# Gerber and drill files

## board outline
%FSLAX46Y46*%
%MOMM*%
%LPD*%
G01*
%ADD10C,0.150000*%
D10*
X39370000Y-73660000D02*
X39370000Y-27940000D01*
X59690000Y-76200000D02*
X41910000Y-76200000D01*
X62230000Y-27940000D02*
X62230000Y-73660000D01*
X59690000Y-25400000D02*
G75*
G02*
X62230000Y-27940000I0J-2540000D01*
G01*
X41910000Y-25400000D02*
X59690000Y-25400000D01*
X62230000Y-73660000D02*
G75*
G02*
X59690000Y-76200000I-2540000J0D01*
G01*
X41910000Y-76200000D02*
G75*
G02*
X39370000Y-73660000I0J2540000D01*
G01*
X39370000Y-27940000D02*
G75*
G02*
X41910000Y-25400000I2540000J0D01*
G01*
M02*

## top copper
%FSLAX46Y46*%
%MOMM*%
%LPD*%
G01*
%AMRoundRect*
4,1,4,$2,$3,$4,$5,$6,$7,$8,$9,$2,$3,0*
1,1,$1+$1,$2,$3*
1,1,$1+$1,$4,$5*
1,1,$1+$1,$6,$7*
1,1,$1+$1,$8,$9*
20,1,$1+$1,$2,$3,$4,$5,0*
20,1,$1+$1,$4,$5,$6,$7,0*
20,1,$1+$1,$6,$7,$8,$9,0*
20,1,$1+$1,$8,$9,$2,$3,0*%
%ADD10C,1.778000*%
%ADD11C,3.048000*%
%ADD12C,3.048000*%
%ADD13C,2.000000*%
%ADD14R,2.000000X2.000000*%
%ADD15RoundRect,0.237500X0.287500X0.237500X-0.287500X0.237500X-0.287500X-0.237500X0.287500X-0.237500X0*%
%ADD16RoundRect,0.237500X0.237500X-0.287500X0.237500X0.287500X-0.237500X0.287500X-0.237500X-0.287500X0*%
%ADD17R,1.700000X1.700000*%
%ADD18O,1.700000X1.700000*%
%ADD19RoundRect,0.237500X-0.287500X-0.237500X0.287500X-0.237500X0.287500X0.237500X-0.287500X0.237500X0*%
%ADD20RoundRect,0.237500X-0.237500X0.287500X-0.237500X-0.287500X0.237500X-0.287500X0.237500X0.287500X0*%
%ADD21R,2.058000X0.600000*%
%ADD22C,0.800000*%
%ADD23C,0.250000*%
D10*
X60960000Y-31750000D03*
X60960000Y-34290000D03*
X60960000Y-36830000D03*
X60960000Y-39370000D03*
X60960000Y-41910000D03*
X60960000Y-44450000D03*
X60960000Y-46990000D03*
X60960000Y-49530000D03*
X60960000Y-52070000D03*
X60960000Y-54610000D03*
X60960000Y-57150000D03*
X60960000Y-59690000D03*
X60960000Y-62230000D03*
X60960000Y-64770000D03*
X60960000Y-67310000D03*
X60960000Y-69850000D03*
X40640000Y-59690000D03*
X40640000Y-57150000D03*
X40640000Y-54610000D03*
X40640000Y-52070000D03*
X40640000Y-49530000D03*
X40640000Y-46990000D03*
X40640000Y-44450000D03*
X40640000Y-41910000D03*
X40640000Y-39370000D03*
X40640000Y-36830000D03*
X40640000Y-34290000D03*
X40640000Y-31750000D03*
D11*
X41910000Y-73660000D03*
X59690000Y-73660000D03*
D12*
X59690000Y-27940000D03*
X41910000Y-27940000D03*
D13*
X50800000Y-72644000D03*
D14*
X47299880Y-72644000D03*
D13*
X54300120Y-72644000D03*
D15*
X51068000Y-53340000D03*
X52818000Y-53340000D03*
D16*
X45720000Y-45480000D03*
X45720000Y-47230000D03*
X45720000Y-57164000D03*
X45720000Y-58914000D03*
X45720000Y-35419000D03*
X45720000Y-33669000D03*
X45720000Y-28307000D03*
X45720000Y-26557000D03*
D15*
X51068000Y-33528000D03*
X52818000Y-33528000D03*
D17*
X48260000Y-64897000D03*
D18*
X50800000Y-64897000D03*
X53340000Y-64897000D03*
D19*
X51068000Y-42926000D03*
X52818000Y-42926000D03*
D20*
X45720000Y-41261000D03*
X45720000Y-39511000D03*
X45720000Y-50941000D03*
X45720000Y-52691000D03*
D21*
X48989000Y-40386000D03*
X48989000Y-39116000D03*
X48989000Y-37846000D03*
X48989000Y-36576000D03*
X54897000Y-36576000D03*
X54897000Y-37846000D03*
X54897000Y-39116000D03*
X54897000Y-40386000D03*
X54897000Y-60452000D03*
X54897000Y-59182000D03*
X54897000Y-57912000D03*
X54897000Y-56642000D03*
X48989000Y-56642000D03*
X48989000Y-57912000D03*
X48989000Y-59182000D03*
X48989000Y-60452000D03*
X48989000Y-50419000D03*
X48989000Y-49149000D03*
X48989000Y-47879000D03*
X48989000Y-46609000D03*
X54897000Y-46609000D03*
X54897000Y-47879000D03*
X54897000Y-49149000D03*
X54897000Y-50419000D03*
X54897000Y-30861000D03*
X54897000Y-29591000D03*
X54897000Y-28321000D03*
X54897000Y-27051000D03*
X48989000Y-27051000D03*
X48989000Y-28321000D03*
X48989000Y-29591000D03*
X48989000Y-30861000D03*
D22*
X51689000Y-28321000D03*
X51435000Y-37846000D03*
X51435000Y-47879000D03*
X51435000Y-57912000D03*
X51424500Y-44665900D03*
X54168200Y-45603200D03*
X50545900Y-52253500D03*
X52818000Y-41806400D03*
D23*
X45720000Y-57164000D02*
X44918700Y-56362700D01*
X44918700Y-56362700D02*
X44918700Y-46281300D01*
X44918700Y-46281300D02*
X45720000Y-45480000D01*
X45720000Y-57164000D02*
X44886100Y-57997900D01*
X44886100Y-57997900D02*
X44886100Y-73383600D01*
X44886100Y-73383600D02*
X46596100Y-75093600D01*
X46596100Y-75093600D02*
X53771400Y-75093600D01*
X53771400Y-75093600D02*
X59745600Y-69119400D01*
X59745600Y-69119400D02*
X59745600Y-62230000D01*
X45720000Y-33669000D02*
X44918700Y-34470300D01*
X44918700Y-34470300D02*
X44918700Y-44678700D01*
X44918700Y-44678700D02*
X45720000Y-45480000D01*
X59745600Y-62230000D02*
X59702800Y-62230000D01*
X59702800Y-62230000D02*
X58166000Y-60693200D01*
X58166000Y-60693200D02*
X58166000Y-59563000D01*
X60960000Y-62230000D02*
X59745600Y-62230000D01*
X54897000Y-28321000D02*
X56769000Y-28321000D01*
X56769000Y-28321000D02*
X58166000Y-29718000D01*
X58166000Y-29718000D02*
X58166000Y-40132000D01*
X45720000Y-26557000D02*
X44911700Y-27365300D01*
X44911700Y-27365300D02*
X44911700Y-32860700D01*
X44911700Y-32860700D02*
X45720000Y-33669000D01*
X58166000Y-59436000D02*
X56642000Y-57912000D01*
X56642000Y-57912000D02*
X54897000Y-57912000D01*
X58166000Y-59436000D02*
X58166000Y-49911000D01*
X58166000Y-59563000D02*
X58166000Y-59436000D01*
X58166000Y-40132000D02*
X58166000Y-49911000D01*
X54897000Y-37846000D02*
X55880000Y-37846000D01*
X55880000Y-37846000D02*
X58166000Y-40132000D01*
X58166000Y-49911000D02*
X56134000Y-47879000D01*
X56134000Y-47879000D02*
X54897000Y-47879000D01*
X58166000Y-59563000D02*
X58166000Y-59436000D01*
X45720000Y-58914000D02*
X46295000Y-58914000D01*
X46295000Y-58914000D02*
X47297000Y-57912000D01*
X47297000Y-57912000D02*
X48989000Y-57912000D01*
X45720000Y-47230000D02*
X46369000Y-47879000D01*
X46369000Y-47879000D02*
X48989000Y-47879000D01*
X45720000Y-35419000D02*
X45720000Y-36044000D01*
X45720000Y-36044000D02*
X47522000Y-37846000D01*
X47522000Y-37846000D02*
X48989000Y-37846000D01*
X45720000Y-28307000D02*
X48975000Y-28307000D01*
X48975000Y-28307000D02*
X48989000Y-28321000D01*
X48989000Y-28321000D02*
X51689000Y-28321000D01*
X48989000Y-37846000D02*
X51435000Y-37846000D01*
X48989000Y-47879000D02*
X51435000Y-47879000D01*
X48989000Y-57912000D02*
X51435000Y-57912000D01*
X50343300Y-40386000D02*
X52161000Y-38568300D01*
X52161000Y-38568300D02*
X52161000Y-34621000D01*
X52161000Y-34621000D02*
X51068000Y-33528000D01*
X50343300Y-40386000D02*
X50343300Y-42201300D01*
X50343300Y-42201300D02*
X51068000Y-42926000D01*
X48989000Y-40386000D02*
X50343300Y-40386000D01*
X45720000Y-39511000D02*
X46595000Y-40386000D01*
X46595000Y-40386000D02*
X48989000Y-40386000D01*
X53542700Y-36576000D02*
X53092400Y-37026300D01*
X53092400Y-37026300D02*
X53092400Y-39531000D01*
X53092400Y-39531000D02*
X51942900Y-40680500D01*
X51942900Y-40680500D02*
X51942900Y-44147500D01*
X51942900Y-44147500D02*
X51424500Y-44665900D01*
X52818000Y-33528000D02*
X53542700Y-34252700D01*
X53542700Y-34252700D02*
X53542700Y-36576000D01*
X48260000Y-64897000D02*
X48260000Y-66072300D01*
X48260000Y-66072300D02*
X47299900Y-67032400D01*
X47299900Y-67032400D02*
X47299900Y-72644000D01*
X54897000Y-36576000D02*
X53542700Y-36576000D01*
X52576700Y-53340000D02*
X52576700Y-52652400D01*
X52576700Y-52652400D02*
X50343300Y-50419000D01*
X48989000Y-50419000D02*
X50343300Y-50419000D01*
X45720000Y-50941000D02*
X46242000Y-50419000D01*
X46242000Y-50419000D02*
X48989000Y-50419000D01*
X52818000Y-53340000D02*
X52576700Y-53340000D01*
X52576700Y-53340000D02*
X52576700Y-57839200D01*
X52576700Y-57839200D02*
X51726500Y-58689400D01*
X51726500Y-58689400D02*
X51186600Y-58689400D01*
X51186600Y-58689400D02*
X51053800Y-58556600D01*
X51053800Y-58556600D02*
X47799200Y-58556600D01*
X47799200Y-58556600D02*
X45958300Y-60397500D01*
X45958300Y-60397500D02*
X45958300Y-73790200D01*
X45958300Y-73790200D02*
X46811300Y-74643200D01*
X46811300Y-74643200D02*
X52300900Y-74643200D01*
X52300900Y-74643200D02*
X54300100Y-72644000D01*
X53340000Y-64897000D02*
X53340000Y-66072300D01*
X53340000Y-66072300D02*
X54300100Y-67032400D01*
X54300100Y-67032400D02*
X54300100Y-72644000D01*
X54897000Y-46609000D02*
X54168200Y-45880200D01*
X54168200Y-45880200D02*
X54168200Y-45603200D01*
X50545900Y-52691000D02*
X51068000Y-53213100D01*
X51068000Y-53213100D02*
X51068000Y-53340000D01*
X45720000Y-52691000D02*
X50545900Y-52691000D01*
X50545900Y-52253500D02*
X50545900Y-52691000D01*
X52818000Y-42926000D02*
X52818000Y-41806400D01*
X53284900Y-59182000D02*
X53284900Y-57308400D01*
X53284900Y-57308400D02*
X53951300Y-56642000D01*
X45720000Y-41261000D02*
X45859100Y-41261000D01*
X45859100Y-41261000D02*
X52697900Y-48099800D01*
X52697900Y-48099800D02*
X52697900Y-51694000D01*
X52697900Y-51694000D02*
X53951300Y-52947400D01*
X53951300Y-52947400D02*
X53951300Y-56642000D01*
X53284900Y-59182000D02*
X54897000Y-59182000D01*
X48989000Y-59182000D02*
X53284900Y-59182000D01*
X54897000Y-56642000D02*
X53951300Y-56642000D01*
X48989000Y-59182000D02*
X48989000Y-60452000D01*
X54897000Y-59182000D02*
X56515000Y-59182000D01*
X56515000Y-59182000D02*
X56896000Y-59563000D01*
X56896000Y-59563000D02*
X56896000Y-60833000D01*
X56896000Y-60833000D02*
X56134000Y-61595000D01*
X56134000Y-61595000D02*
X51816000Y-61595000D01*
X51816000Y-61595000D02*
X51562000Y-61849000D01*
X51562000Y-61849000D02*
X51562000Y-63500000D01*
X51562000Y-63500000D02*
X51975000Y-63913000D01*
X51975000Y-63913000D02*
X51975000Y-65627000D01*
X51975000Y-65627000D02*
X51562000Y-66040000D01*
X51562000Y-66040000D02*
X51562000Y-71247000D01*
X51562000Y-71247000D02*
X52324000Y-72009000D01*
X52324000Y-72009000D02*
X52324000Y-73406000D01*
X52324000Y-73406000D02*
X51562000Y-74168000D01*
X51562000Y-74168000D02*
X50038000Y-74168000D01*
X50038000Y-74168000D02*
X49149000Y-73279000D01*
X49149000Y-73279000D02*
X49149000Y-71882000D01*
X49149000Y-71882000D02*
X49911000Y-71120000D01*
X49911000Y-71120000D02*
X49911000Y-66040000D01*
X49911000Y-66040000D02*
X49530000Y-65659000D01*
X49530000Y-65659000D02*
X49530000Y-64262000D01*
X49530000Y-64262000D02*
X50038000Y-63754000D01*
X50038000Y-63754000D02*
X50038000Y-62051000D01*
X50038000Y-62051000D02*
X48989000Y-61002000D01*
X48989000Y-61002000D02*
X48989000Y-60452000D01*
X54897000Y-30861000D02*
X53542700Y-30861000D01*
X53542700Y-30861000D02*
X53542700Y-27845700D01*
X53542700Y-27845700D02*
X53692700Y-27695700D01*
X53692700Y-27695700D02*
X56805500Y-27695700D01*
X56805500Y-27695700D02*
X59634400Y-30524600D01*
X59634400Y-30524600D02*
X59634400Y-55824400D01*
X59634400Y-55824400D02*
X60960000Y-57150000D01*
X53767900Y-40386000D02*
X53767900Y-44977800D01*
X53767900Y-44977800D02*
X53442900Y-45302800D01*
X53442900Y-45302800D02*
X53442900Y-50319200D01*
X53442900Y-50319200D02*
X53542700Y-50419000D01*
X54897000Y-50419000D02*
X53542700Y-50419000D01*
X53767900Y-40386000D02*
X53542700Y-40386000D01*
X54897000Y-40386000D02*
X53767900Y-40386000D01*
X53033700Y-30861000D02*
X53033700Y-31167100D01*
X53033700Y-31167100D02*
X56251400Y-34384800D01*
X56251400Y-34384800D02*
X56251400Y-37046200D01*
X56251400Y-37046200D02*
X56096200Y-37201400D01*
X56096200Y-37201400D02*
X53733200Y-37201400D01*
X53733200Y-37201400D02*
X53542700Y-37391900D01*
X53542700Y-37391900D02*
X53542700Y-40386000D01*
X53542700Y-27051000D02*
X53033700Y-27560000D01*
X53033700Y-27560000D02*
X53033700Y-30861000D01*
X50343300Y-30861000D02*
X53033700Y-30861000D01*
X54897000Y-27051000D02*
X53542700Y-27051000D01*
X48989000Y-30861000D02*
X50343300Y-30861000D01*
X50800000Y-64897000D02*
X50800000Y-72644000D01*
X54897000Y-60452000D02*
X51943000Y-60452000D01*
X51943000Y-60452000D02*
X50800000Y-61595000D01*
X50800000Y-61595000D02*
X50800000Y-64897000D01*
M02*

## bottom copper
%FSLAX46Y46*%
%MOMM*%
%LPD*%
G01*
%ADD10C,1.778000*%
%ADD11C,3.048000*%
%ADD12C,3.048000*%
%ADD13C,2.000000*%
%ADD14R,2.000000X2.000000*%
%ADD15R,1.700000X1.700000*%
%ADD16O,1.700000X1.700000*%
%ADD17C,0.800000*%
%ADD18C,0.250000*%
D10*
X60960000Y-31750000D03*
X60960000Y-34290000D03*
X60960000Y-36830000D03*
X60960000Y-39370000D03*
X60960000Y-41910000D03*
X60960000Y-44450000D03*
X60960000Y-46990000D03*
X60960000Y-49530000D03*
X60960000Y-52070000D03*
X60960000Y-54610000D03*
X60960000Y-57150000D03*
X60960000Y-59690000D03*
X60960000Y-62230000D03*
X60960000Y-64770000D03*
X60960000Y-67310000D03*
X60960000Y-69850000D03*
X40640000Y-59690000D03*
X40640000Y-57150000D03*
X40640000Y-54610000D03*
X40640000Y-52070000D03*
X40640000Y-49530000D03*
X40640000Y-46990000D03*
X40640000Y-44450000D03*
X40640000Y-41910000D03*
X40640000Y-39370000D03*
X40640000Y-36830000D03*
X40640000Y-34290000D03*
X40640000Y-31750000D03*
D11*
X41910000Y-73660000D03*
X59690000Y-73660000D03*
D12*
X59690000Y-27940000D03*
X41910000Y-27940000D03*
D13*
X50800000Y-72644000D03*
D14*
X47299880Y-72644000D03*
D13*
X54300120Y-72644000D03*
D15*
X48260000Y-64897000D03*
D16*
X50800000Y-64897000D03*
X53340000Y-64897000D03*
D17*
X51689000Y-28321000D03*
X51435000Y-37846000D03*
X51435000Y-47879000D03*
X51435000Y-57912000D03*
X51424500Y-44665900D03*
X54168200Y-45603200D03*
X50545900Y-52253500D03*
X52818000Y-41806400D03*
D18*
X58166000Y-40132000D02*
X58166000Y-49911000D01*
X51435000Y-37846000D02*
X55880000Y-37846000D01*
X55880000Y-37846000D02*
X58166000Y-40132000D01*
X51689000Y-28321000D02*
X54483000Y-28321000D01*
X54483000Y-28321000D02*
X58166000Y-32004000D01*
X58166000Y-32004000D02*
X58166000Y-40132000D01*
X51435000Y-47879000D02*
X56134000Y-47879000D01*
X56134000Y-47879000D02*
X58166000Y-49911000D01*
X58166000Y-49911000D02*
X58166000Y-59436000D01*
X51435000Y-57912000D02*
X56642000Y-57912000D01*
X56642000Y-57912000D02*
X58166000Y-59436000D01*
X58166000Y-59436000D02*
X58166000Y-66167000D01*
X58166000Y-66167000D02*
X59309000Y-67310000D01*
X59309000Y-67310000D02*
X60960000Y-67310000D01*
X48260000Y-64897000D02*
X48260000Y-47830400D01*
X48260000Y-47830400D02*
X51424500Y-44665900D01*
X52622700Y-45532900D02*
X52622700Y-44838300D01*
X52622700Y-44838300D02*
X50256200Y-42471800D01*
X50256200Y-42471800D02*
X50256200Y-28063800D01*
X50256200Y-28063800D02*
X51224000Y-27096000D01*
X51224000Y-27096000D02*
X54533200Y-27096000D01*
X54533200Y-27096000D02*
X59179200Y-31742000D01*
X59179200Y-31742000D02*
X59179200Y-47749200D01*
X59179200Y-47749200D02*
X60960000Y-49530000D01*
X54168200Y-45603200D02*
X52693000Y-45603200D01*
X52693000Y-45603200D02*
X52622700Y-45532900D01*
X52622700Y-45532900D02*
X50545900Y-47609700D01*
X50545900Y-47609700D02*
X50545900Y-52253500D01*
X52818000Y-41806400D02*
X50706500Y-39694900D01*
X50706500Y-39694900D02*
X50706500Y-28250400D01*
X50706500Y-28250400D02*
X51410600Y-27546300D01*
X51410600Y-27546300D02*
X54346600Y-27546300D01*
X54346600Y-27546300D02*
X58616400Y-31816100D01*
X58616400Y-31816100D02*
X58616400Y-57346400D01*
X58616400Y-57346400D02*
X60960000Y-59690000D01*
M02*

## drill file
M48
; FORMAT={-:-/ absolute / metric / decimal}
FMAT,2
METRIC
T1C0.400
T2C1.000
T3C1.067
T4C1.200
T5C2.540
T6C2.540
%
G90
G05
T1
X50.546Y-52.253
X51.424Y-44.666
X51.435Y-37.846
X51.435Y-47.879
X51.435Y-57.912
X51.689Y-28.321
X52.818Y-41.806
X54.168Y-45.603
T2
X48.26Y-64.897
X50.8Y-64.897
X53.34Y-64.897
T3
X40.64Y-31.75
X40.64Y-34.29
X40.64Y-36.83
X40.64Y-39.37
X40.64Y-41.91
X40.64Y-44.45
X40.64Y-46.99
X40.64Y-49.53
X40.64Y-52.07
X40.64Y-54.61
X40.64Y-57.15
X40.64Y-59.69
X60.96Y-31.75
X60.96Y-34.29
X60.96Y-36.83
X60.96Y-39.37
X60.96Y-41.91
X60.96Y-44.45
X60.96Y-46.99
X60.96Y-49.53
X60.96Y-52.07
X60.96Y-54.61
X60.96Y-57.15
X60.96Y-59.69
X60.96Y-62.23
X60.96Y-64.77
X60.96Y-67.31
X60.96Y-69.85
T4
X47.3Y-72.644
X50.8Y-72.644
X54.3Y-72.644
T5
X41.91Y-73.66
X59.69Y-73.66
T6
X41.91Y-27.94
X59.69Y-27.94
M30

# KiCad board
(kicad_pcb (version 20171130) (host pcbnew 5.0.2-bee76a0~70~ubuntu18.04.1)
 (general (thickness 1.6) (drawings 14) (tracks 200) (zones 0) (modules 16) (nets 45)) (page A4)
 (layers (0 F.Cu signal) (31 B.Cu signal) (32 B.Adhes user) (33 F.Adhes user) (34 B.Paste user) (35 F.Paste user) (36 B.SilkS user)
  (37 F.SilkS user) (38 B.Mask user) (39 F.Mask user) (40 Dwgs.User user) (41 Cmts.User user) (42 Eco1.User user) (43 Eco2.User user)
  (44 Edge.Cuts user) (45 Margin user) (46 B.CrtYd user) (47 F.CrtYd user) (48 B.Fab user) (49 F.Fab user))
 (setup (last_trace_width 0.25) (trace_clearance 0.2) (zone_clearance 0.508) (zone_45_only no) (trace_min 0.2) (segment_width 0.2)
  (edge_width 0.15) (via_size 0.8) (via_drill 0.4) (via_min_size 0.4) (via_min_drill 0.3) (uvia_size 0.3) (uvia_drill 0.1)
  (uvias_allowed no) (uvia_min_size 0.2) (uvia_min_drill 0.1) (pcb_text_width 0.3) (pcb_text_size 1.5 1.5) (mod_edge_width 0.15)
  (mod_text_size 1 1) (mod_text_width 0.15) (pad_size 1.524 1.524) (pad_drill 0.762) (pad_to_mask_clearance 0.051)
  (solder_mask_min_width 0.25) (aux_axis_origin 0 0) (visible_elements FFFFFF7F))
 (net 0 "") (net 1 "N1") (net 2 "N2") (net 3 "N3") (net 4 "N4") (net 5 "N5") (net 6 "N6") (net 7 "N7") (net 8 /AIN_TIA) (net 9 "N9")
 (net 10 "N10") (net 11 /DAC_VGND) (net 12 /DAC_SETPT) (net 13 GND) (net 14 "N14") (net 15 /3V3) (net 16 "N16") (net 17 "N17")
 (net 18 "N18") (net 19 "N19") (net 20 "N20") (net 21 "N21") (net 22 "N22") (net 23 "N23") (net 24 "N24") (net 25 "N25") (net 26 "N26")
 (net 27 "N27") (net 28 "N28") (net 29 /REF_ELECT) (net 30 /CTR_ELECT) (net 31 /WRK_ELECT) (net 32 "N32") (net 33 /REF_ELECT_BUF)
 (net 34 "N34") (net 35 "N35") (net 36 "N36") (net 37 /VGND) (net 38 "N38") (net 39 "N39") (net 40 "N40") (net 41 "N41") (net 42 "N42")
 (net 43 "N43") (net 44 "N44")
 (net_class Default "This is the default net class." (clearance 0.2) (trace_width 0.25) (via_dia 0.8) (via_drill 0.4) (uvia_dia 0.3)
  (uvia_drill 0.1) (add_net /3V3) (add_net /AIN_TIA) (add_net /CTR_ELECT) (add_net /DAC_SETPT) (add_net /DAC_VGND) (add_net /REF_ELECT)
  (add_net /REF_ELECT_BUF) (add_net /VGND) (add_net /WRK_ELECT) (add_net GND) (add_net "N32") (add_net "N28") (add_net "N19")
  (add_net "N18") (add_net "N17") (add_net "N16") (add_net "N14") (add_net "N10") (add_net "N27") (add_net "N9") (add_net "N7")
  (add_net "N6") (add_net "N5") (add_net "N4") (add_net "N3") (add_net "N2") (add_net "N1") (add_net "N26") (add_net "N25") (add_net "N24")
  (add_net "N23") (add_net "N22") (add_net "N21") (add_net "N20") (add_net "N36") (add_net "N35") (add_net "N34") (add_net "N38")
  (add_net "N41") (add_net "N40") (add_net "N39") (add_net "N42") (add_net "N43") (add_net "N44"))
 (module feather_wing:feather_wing (layer F.Cu) (at 50.8 50.8)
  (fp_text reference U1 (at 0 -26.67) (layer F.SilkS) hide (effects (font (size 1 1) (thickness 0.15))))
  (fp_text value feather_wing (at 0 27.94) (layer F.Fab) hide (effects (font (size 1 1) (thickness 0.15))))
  (pad 28 thru_hole circle (at 10.16 -19.05) (size 1.778 1.778) (drill 1.0668) (layers *.Cu *.Mask) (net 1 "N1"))
  (pad 27 thru_hole circle (at 10.16 -16.51) (size 1.778 1.778) (drill 1.0668) (layers *.Cu *.Mask) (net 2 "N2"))
  (pad 26 thru_hole circle (at 10.16 -13.97) (size 1.778 1.778) (drill 1.0668) (layers *.Cu *.Mask) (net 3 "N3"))
  (pad 25 thru_hole circle (at 10.16 -11.43) (size 1.778 1.778) (drill 1.0668) (layers *.Cu *.Mask) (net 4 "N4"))
  (pad 24 thru_hole circle (at 10.16 -8.89) (size 1.778 1.778) (drill 1.0668) (layers *.Cu *.Mask) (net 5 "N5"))
  (pad 23 thru_hole circle (at 10.16 -6.35) (size 1.778 1.778) (drill 1.0668) (layers *.Cu *.Mask) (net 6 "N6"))
  (pad 22 thru_hole circle (at 10.16 -3.81) (size 1.778 1.778) (drill 1.0668) (layers *.Cu *.Mask) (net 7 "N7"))
  (pad 21 thru_hole circle (at 10.16 -1.27) (size 1.778 1.778) (drill 1.0668) (layers *.Cu *.Mask) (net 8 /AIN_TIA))
  (pad 20 thru_hole circle (at 10.16 1.27) (size 1.778 1.778) (drill 1.0668) (layers *.Cu *.Mask) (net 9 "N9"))
  (pad 19 thru_hole circle (at 10.16 3.81) (size 1.778 1.778) (drill 1.0668) (layers *.Cu *.Mask) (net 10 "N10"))
  (pad 18 thru_hole circle (at 10.16 6.35) (size 1.778 1.778) (drill 1.0668) (layers *.Cu *.Mask) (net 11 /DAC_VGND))
  (pad 17 thru_hole circle (at 10.16 8.89) (size 1.778 1.778) (drill 1.0668) (layers *.Cu *.Mask) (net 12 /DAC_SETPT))
  (pad 16 thru_hole circle (at 10.16 11.43) (size 1.778 1.778) (drill 1.0668) (layers *.Cu *.Mask) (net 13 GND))
  (pad 15 thru_hole circle (at 10.16 13.97) (size 1.778 1.778) (drill 1.0668) (layers *.Cu *.Mask) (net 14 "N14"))
  (pad 14 thru_hole circle (at 10.16 16.51) (size 1.778 1.778) (drill 1.0668) (layers *.Cu *.Mask) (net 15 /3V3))
  (pad 13 thru_hole circle (at 10.16 19.05) (size 1.778 1.778) (drill 1.0668) (layers *.Cu *.Mask) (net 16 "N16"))
  (pad 12 thru_hole circle (at -10.16 8.89) (size 1.778 1.778) (drill 1.0668) (layers *.Cu *.Mask) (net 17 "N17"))
  (pad 11 thru_hole circle (at -10.16 6.35) (size 1.778 1.778) (drill 1.0668) (layers *.Cu *.Mask) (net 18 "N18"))
  (pad 10 thru_hole circle (at -10.16 3.81) (size 1.778 1.778) (drill 1.0668) (layers *.Cu *.Mask) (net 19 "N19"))
  (pad 9 thru_hole circle (at -10.16 1.27) (size 1.778 1.778) (drill 1.0668) (layers *.Cu *.Mask) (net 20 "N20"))
  (pad 8 thru_hole circle (at -10.16 -1.27) (size 1.778 1.778) (drill 1.0668) (layers *.Cu *.Mask) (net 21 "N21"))
  (pad 7 thru_hole circle (at -10.16 -3.81) (size 1.778 1.778) (drill 1.0668) (layers *.Cu *.Mask) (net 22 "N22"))
  (pad 6 thru_hole circle (at -10.16 -6.35) (size 1.778 1.778) (drill 1.0668) (layers *.Cu *.Mask) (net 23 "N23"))
  (pad 5 thru_hole circle (at -10.16 -8.89) (size 1.778 1.778) (drill 1.0668) (layers *.Cu *.Mask) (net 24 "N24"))
  (pad 4 thru_hole circle (at -10.16 -11.43) (size 1.778 1.778) (drill 1.0668) (layers *.Cu *.Mask) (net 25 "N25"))
  (pad 3 thru_hole circle (at -10.16 -13.97) (size 1.778 1.778) (drill 1.0668) (layers *.Cu *.Mask) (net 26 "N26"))
  (pad 2 thru_hole circle (at -10.16 -16.51) (size 1.778 1.778) (drill 1.0668) (layers *.Cu *.Mask) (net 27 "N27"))
  (pad 1 thru_hole circle (at -10.16 -19.05) (size 1.778 1.778) (drill 1.0668) (layers *.Cu *.Mask) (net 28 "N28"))
  (pad "" thru_hole circle (at -8.89 22.86) (size 3.048 3.048) (drill 2.54) (layers *.Cu *.Mask))
  (pad "" thru_hole circle (at 8.89 22.86) (size 3.048 3.048) (drill 2.54) (layers *.Cu *.Mask))
  (pad "" np_thru_hole circle (at 8.89 -22.86) (size 3.048 3.048) (drill 2.54) (layers *.Cu *.Mask))
  (pad "" np_thru_hole circle (at -8.89 -22.86) (size 3.048 3.048) (drill 2.54) (layers *.Cu *.Mask)))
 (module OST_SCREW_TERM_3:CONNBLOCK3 (layer F.Cu) (at 50.8 72.644)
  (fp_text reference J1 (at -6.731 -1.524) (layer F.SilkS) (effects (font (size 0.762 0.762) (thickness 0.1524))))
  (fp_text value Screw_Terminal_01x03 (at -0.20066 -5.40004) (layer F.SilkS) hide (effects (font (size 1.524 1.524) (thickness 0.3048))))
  (pad 2 thru_hole circle (at 0 0) (size 2 2) (drill 1.2) (layers *.Cu *.Mask) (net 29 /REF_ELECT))
  (pad 1 thru_hole rect (at -3.50012 0) (size 2 2) (drill 1.2) (layers *.Cu *.Mask) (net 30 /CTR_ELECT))
  (pad 3 thru_hole circle (at 3.50012 0) (size 2 2) (drill 1.2) (layers *.Cu *.Mask) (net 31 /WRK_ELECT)))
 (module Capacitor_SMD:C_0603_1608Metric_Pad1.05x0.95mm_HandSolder (layer F.Cu) (at 51.943 53.34 180)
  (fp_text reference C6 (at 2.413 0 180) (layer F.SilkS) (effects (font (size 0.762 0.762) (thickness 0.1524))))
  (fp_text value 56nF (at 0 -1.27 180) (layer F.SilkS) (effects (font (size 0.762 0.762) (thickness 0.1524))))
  (pad 2 smd roundrect (at 0.875 0 180) (size 1.05 0.95) (layers F.Cu F.Paste F.Mask) (roundrect_rratio 0.25) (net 8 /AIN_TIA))
  (pad 1 smd roundrect (at -0.875 0 180) (size 1.05 0.95) (layers F.Cu F.Paste F.Mask) (roundrect_rratio 0.25) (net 31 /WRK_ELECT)))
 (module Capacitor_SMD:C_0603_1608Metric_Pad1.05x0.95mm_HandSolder (layer F.Cu) (at 45.72 46.355 90)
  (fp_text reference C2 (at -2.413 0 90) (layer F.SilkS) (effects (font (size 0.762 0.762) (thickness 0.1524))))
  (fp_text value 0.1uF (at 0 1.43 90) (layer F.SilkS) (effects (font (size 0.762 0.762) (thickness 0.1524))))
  (pad 2 smd roundrect (at 0.875 0 90) (size 1.05 0.95) (layers F.Cu F.Paste F.Mask) (roundrect_rratio 0.25) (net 13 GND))
  (pad 1 smd roundrect (at -0.875 0 90) (size 1.05 0.95) (layers F.Cu F.Paste F.Mask) (roundrect_rratio 0.25) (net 15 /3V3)))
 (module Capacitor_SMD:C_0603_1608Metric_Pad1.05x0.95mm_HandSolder (layer F.Cu) (at 45.72 58.039 90)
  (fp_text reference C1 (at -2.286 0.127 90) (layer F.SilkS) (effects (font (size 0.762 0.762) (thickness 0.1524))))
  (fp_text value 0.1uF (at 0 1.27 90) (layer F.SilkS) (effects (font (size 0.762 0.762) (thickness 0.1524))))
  (pad 2 smd roundrect (at 0.875 0 90) (size 1.05 0.95) (layers F.Cu F.Paste F.Mask) (roundrect_rratio 0.25) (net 13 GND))
  (pad 1 smd roundrect (at -0.875 0 90) (size 1.05 0.95) (layers F.Cu F.Paste F.Mask) (roundrect_rratio 0.25) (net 15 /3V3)))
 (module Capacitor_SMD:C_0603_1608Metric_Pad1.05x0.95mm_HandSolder (layer F.Cu) (at 45.72 34.544 90)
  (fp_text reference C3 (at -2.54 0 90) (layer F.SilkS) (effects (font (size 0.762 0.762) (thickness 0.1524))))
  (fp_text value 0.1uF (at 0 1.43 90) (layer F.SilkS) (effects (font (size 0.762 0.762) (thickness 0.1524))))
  (pad 1 smd roundrect (at -0.875 0 90) (size 1.05 0.95) (layers F.Cu F.Paste F.Mask) (roundrect_rratio 0.25) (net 15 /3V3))
  (pad 2 smd roundrect (at 0.875 0 90) (size 1.05 0.95) (layers F.Cu F.Paste F.Mask) (roundrect_rratio 0.25) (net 13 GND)))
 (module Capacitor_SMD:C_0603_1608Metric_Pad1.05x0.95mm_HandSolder (layer F.Cu) (at 45.72 27.432 90)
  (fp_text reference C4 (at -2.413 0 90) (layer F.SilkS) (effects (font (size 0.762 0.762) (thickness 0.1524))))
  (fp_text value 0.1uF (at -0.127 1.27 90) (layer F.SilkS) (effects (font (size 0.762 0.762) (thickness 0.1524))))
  (pad 1 smd roundrect (at -0.875 0 90) (size 1.05 0.95) (layers F.Cu F.Paste F.Mask) (roundrect_rratio 0.25) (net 15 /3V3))
  (pad 2 smd roundrect (at 0.875 0 90) (size 1.05 0.95) (layers F.Cu F.Paste F.Mask) (roundrect_rratio 0.25) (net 13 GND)))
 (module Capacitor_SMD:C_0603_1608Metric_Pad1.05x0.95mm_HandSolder (layer F.Cu) (at 51.943 33.528 180)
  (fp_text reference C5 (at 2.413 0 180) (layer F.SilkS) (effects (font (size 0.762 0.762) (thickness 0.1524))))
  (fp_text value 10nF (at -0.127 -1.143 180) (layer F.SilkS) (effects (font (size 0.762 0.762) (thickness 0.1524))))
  (pad 2 smd roundrect (at 0.875 0 180) (size 1.05 0.95) (layers F.Cu F.Paste F.Mask) (roundrect_rratio 0.25) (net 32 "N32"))
  (pad 1 smd roundrect (at -0.875 0 180) (size 1.05 0.95) (layers F.Cu F.Paste F.Mask) (roundrect_rratio 0.25) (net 30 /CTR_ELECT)))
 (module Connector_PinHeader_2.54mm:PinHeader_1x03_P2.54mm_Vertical (layer F.Cu) (at 48.26 64.897 90)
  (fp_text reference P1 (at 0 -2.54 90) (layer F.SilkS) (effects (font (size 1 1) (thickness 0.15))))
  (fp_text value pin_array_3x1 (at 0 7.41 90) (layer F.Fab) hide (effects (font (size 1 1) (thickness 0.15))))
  (pad 1 thru_hole rect (at 0 0 90) (size 1.7 1.7) (drill 1) (layers *.Cu *.Mask) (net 30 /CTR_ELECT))
  (pad 2 thru_hole oval (at 0 2.54 90) (size 1.7 1.7) (drill 1) (layers *.Cu *.Mask) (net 29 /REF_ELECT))
  (pad 3 thru_hole oval (at 0 5.08 90) (size 1.7 1.7) (drill 1) (layers *.Cu *.Mask) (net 31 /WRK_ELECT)))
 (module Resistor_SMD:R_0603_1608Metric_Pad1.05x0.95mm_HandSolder (layer F.Cu) (at 51.943 42.926)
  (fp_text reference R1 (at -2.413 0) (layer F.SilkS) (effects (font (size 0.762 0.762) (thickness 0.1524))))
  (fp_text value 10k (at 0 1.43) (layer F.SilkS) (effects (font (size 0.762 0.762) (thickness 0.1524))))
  (pad 1 smd roundrect (at -0.875 0) (size 1.05 0.95) (layers F.Cu F.Paste F.Mask) (roundrect_rratio 0.25) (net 32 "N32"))
  (pad 2 smd roundrect (at 0.875 0) (size 1.05 0.95) (layers F.Cu F.Paste F.Mask) (roundrect_rratio 0.25) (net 12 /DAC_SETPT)))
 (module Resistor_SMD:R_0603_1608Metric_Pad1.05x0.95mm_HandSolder (layer F.Cu) (at 45.72 40.386 270)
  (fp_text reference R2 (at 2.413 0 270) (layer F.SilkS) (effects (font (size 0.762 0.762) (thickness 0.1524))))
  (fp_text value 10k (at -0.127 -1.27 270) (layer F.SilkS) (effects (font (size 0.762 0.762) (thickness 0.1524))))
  (pad 2 smd roundrect (at 0.875 0 270) (size 1.05 0.95) (layers F.Cu F.Paste F.Mask) (roundrect_rratio 0.25) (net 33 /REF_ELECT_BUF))
  (pad 1 smd roundrect (at -0.875 0 270) (size 1.05 0.95) (layers F.Cu F.Paste F.Mask) (roundrect_rratio 0.25) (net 32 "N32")))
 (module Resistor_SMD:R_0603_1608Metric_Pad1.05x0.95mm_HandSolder (layer F.Cu) (at 45.72 51.816 270)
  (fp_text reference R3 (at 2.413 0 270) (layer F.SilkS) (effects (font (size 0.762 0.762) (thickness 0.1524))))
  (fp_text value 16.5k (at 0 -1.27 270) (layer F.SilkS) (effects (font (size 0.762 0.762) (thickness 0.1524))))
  (pad 1 smd roundrect (at -0.875 0 270) (size 1.05 0.95) (layers F.Cu F.Paste F.Mask) (roundrect_rratio 0.25) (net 31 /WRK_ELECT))
  (pad 2 smd roundrect (at 0.875 0 270) (size 1.05 0.95) (layers F.Cu F.Paste F.Mask) (roundrect_rratio 0.25) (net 8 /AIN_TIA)))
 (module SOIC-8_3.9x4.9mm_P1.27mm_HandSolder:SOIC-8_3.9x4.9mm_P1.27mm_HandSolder (layer F.Cu) (at 51.943 38.481 180)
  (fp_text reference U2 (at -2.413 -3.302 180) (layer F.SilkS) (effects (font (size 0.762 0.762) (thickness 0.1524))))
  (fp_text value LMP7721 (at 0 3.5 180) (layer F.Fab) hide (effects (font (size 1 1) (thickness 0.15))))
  (pad 8 smd rect (at 2.954 -1.905 180) (size 2.058 0.6) (layers F.Cu F.Paste F.Mask) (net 32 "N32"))
  (pad 7 smd rect (at 2.954 -0.635 180) (size 2.058 0.6) (layers F.Cu F.Paste F.Mask) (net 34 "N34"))
  (pad 6 smd rect (at 2.954 0.635 180) (size 2.058 0.6) (layers F.Cu F.Paste F.Mask) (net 15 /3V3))
  (pad 5 smd rect (at 2.954 1.905 180) (size 2.058 0.6) (layers F.Cu F.Paste F.Mask) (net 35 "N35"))
  (pad 4 smd rect (at -2.954 1.905 180) (size 2.058 0.6) (layers F.Cu F.Paste F.Mask) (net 30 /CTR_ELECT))
  (pad 3 smd rect (at -2.954 0.635 180) (size 2.058 0.6) (layers F.Cu F.Paste F.Mask) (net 13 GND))
  (pad 2 smd rect (at -2.954 -0.635 180) (size 2.058 0.6) (layers F.Cu F.Paste F.Mask) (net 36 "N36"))
  (pad 1 smd rect (at -2.954 -1.905 180) (size 2.058 0.6) (layers F.Cu F.Paste F.Mask) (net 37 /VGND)))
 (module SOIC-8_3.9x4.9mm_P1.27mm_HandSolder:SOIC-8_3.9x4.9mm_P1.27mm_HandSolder (layer F.Cu) (at 51.943 58.547 180)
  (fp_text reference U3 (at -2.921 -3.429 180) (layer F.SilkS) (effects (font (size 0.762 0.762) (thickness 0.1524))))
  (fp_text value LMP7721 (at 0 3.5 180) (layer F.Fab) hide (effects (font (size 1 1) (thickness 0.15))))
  (pad 1 smd rect (at -2.954 -1.905 180) (size 2.058 0.6) (layers F.Cu F.Paste F.Mask) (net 29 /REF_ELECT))
  (pad 2 smd rect (at -2.954 -0.635 180) (size 2.058 0.6) (layers F.Cu F.Paste F.Mask) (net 33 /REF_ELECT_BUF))
  (pad 3 smd rect (at -2.954 0.635 180) (size 2.058 0.6) (layers F.Cu F.Paste F.Mask) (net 13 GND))
  (pad 4 smd rect (at -2.954 1.905 180) (size 2.058 0.6) (layers F.Cu F.Paste F.Mask) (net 33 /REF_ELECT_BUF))
  (pad 5 smd rect (at 2.954 1.905 180) (size 2.058 0.6) (layers F.Cu F.Paste F.Mask) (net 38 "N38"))
  (pad 6 smd rect (at 2.954 0.635 180) (size 2.058 0.6) (layers F.Cu F.Paste F.Mask) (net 15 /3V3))
  (pad 7 smd rect (at 2.954 -0.635 180) (size 2.058 0.6) (layers F.Cu F.Paste F.Mask) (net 33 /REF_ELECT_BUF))
  (pad 8 smd rect (at 2.954 -1.905 180) (size 2.058 0.6) (layers F.Cu F.Paste F.Mask) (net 33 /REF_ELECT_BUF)))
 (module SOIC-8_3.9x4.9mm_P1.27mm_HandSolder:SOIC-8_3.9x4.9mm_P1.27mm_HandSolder (layer F.Cu) (at 51.943 48.514 180)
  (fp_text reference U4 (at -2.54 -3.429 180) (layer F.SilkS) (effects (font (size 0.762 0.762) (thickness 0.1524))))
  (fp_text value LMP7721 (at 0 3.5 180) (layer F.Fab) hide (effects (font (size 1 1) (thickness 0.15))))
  (pad 8 smd rect (at 2.954 -1.905 180) (size 2.058 0.6) (layers F.Cu F.Paste F.Mask) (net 31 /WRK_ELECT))
  (pad 7 smd rect (at 2.954 -0.635 180) (size 2.058 0.6) (layers F.Cu F.Paste F.Mask) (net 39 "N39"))
  (pad 6 smd rect (at 2.954 0.635 180) (size 2.058 0.6) (layers F.Cu F.Paste F.Mask) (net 15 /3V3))
  (pad 5 smd rect (at 2.954 1.905 180) (size 2.058 0.6) (layers F.Cu F.Paste F.Mask) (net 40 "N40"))
  (pad 4 smd rect (at -2.954 1.905 180) (size 2.058 0.6) (layers F.Cu F.Paste F.Mask) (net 8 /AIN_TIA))
  (pad 3 smd rect (at -2.954 0.635 180) (size 2.058 0.6) (layers F.Cu F.Paste F.Mask) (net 13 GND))
  (pad 2 smd rect (at -2.954 -0.635 180) (size 2.058 0.6) (layers F.Cu F.Paste F.Mask) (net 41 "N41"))
  (pad 1 smd rect (at -2.954 -1.905 180) (size 2.058 0.6) (layers F.Cu F.Paste F.Mask) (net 37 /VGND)))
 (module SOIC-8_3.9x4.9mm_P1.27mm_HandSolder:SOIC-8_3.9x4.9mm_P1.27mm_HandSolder (layer F.Cu) (at 51.943 28.956 180)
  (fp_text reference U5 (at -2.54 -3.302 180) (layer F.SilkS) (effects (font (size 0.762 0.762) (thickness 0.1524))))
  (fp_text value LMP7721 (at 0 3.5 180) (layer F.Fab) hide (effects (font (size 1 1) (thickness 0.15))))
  (pad 1 smd rect (at -2.954 -1.905 180) (size 2.058 0.6) (layers F.Cu F.Paste F.Mask) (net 11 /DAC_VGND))
  (pad 2 smd rect (at -2.954 -0.635 180) (size 2.058 0.6) (layers F.Cu F.Paste F.Mask) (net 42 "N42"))
  (pad 3 smd rect (at -2.954 0.635 180) (size 2.058 0.6) (layers F.Cu F.Paste F.Mask) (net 13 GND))
  (pad 4 smd rect (at -2.954 1.905 180) (size 2.058 0.6) (layers F.Cu F.Paste F.Mask) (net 37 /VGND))
  (pad 5 smd rect (at 2.954 1.905 180) (size 2.058 0.6) (layers F.Cu F.Paste F.Mask) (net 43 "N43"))
  (pad 6 smd rect (at 2.954 0.635 180) (size 2.058 0.6) (layers F.Cu F.Paste F.Mask) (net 15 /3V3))
  (pad 7 smd rect (at 2.954 -0.635 180) (size 2.058 0.6) (layers F.Cu F.Paste F.Mask) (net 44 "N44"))
  (pad 8 smd rect (at 2.954 -1.905 180) (size 2.058 0.6) (layers F.Cu F.Paste F.Mask) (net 37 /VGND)))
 (gr_line (start 39.37 73.66) (end 39.37 27.94) (layer Edge.Cuts) (width 0.15))
 (gr_line (start 59.69 76.2) (end 41.91 76.2) (layer Edge.Cuts) (width 0.15))
 (gr_line (start 62.23 27.94) (end 62.23 73.66) (layer Edge.Cuts) (width 0.15))
 (gr_arc (start 59.69 27.94) (end 62.23 27.94) (angle -90) (layer Edge.Cuts) (width 0.15))
 (gr_line (start 41.91 25.4) (end 59.69 25.4) (layer Edge.Cuts) (width 0.15))
 (gr_arc (start 59.69 73.66) (end 59.69 76.2) (angle -90) (layer Edge.Cuts) (width 0.15))
 (gr_arc (start 41.91 73.66) (end 39.37 73.66) (angle -90) (layer Edge.Cuts) (width 0.15))
 (gr_arc (start 41.91 27.94) (end 41.91 25.4) (angle -90) (layer Edge.Cuts) (width 0.15))
 (segment (start 45.72 57.164) (end 44.9187 56.3627) (width 0.25) (layer F.Cu) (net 13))
 (segment (start 44.9187 56.3627) (end 44.9187 46.2813) (width 0.25) (layer F.Cu) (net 13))
 (segment (start 44.9187 46.2813) (end 45.72 45.48) (width 0.25) (layer F.Cu) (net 13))
 (segment (start 45.72 57.164) (end 44.8861 57.9979) (width 0.25) (layer F.Cu) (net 13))
 (segment (start 44.8861 57.9979) (end 44.8861 73.3836) (width 0.25) (layer F.Cu) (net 13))
 (segment (start 44.8861 73.3836) (end 46.5961 75.0936) (width 0.25) (layer F.Cu) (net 13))
 (segment (start 46.5961 75.0936) (end 53.7714 75.0936) (width 0.25) (layer F.Cu) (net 13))
 (segment (start 53.7714 75.0936) (end 59.7456 69.1194) (width 0.25) (layer F.Cu) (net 13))
 (segment (start 59.7456 69.1194) (end 59.7456 62.23) (width 0.25) (layer F.Cu) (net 13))
 (segment (start 45.72 33.669) (end 44.9187 34.4703) (width 0.25) (layer F.Cu) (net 13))
 (segment (start 44.9187 34.4703) (end 44.9187 44.6787) (width 0.25) (layer F.Cu) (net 13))
 (segment (start 44.9187 44.6787) (end 45.72 45.48) (width 0.25) (layer F.Cu) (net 13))
 (segment (start 59.7456 62.23) (end 59.7028 62.23) (width 0.25) (layer F.Cu) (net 13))
 (segment (start 59.7028 62.23) (end 58.166 60.6932) (width 0.25) (layer F.Cu) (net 13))
 (segment (start 58.166 60.6932) (end 58.166 59.563) (width 0.25) (layer F.Cu) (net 13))
 (segment (start 60.96 62.23) (end 59.7456 62.23) (width 0.25) (layer F.Cu) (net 13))
 (segment (start 54.897 28.321) (end 56.769 28.321) (width 0.25) (layer F.Cu) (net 13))
 (segment (start 56.769 28.321) (end 58.166 29.718) (width 0.25) (layer F.Cu) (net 13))
 (segment (start 58.166 29.718) (end 58.166 40.132) (width 0.25) (layer F.Cu) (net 13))
 (segment (start 45.72 26.557) (end 44.9117 27.3653) (width 0.25) (layer F.Cu) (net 13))
 (segment (start 44.9117 27.3653) (end 44.9117 32.8607) (width 0.25) (layer F.Cu) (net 13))
 (segment (start 44.9117 32.8607) (end 45.72 33.669) (width 0.25) (layer F.Cu) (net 13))
 (segment (start 58.166 59.436) (end 56.642 57.912) (width 0.25) (layer F.Cu) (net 13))
 (segment (start 56.642 57.912) (end 54.897 57.912) (width 0.25) (layer F.Cu) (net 13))
 (segment (start 58.166 59.436) (end 58.166 49.911) (width 0.25) (layer F.Cu) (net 13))
 (segment (start 58.166 59.563) (end 58.166 59.436) (width 0.25) (layer F.Cu) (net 13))
 (segment (start 58.166 40.132) (end 58.166 49.911) (width 0.25) (layer F.Cu) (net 13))
 (segment (start 54.897 37.846) (end 55.88 37.846) (width 0.25) (layer F.Cu) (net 13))
 (segment (start 55.88 37.846) (end 58.166 40.132) (width 0.25) (layer F.Cu) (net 13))
 (segment (start 58.166 49.911) (end 56.134 47.879) (width 0.25) (layer F.Cu) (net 13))
 (segment (start 56.134 47.879) (end 54.897 47.879) (width 0.25) (layer F.Cu) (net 13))
 (segment (start 58.166 59.563) (end 58.166 59.436) (width 0.25) (layer F.Cu) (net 13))
 (segment (start 58.166 40.132) (end 58.166 49.911) (width 0.25) (layer B.Cu) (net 15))
 (segment (start 51.435 37.846) (end 55.88 37.846) (width 0.25) (layer B.Cu) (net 15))
 (segment (start 55.88 37.846) (end 58.166 40.132) (width 0.25) (layer B.Cu) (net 15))
 (segment (start 45.72 58.914) (end 46.295 58.914) (width 0.25) (layer F.Cu) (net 15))
 (segment (start 46.295 58.914) (end 47.297 57.912) (width 0.25) (layer F.Cu) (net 15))
 (segment (start 47.297 57.912) (end 48.989 57.912) (width 0.25) (layer F.Cu) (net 15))
 (segment (start 45.72 47.23) (end 46.369 47.879) (width 0.25) (layer F.Cu) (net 15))
 (segment (start 46.369 47.879) (end 48.989 47.879) (width 0.25) (layer F.Cu) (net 15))
 (segment (start 45.72 35.419) (end 45.72 36.044) (width 0.25) (layer F.Cu) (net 15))
 (segment (start 45.72 36.044) (end 47.522 37.846) (width 0.25) (layer F.Cu) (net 15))
 (segment (start 47.522 37.846) (end 48.989 37.846) (width 0.25) (layer F.Cu) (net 15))
 (segment (start 45.72 28.307) (end 48.975 28.307) (width 0.25) (layer F.Cu) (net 15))
 (segment (start 48.975 28.307) (end 48.989 28.321) (width 0.25) (layer F.Cu) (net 15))
 (segment (start 51.689 28.321) (end 54.483 28.321) (width 0.25) (layer B.Cu) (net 15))
 (segment (start 54.483 28.321) (end 58.166 32.004) (width 0.25) (layer B.Cu) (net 15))
 (segment (start 58.166 32.004) (end 58.166 40.132) (width 0.25) (layer B.Cu) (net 15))
 (segment (start 48.989 28.321) (end 51.689 28.321) (width 0.25) (layer F.Cu) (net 15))
 (segment (start 48.989 37.846) (end 51.435 37.846) (width 0.25) (layer F.Cu) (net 15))
 (segment (start 51.435 47.879) (end 56.134 47.879) (width 0.25) (layer B.Cu) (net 15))
 (segment (start 56.134 47.879) (end 58.166 49.911) (width 0.25) (layer B.Cu) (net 15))
 (segment (start 58.166 49.911) (end 58.166 59.436) (width 0.25) (layer B.Cu) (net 15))
 (segment (start 48.989 47.879) (end 51.435 47.879) (width 0.25) (layer F.Cu) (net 15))
 (segment (start 51.435 57.912) (end 56.642 57.912) (width 0.25) (layer B.Cu) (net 15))
 (segment (start 56.642 57.912) (end 58.166 59.436) (width 0.25) (layer B.Cu) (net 15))
 (segment (start 58.166 59.436) (end 58.166 66.167) (width 0.25) (layer B.Cu) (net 15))
 (segment (start 58.166 66.167) (end 59.309 67.31) (width 0.25) (layer B.Cu) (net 15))
 (segment (start 59.309 67.31) (end 60.96 67.31) (width 0.25) (layer B.Cu) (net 15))
 (segment (start 48.989 57.912) (end 51.435 57.912) (width 0.25) (layer F.Cu) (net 15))
 (via (at 51.689 28.321) (size 0.8) (layers F.Cu B.Cu) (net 15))
 (via (at 51.435 37.846) (size 0.8) (layers F.Cu B.Cu) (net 15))
 (via (at 51.435 47.879) (size 0.8) (layers F.Cu B.Cu) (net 15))
 (via (at 51.435 57.912) (size 0.8) (layers F.Cu B.Cu) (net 15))
 (segment (start 50.3433 40.386) (end 52.161 38.5683) (width 0.25) (layer F.Cu) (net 32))
 (segment (start 52.161 38.5683) (end 52.161 34.621) (width 0.25) (layer F.Cu) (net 32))
 (segment (start 52.161 34.621) (end 51.068 33.528) (width 0.25) (layer F.Cu) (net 32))
 (segment (start 50.3433 40.386) (end 50.3433 42.2013) (width 0.25) (layer F.Cu) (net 32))
 (segment (start 50.3433 42.2013) (end 51.068 42.926) (width 0.25) (layer F.Cu) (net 32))
 (segment (start 48.989 40.386) (end 50.3433 40.386) (width 0.25) (layer F.Cu) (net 32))
 (segment (start 45.72 39.511) (end 46.595 40.386) (width 0.25) (layer F.Cu) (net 32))
 (segment (start 46.595 40.386) (end 48.989 40.386) (width 0.25) (layer F.Cu) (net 32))
 (segment (start 53.5427 36.576) (end 53.0924 37.0263) (width 0.25) (layer F.Cu) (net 30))
 (segment (start 53.0924 37.0263) (end 53.0924 39.531) (width 0.25) (layer F.Cu) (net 30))
 (segment (start 53.0924 39.531) (end 51.9429 40.6805) (width 0.25) (layer F.Cu) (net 30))
 (segment (start 51.9429 40.6805) (end 51.9429 44.1475) (width 0.25) (layer F.Cu) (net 30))
 (segment (start 51.9429 44.1475) (end 51.4245 44.6659) (width 0.25) (layer F.Cu) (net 30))
 (segment (start 48.26 64.897) (end 48.26 47.8304) (width 0.25) (layer B.Cu) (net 30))
 (segment (start 48.26 47.8304) (end 51.4245 44.6659) (width 0.25) (layer B.Cu) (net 30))
 (segment (start 52.818 33.528) (end 53.5427 34.2527) (width 0.25) (layer F.Cu) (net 30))
 (segment (start 53.5427 34.2527) (end 53.5427 36.576) (width 0.25) (layer F.Cu) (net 30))
 (segment (start 48.26 64.897) (end 48.26 66.0723) (width 0.25) (layer F.Cu) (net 30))
 (segment (start 48.26 66.0723) (end 47.2999 67.0324) (width 0.25) (layer F.Cu) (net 30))
 (segment (start 47.2999 67.0324) (end 47.2999 72.644) (width 0.25) (layer F.Cu) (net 30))
 (segment (start 54.897 36.576) (end 53.5427 36.576) (width 0.25) (layer F.Cu) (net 30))
 (via (at 51.4245 44.6659) (size 0.8) (layers F.Cu B.Cu) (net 30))
 (segment (start 52.5767 53.34) (end 52.5767 52.6524) (width 0.25) (layer F.Cu) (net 31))
 (segment (start 52.5767 52.6524) (end 50.3433 50.419) (width 0.25) (layer F.Cu) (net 31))
 (segment (start 48.989 50.419) (end 50.3433 50.419) (width 0.25) (layer F.Cu) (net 31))
 (segment (start 45.72 50.941) (end 46.242 50.419) (width 0.25) (layer F.Cu) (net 31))
 (segment (start 46.242 50.419) (end 48.989 50.419) (width 0.25) (layer F.Cu) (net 31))
 (segment (start 52.818 53.34) (end 52.5767 53.34) (width 0.25) (layer F.Cu) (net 31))
 (segment (start 52.5767 53.34) (end 52.5767 57.8392) (width 0.25) (layer F.Cu) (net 31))
 (segment (start 52.5767 57.8392) (end 51.7265 58.6894) (width 0.25) (layer F.Cu) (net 31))
 (segment (start 51.7265 58.6894) (end 51.1866 58.6894) (width 0.25) (layer F.Cu) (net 31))
 (segment (start 51.1866 58.6894) (end 51.0538 58.5566) (width 0.25) (layer F.Cu) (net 31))
 (segment (start 51.0538 58.5566) (end 47.7992 58.5566) (width 0.25) (layer F.Cu) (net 31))
 (segment (start 47.7992 58.5566) (end 45.9583 60.3975) (width 0.25) (layer F.Cu) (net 31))
 (segment (start 45.9583 60.3975) (end 45.9583 73.7902) (width 0.25) (layer F.Cu) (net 31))
 (segment (start 45.9583 73.7902) (end 46.8113 74.6432) (width 0.25) (layer F.Cu) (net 31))
 (segment (start 46.8113 74.6432) (end 52.3009 74.6432) (width 0.25) (layer F.Cu) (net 31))
 (segment (start 52.3009 74.6432) (end 54.3001 72.644) (width 0.25) (layer F.Cu) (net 31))
 (segment (start 53.34 64.897) (end 53.34 66.0723) (width 0.25) (layer F.Cu) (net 31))
 (segment (start 53.34 66.0723) (end 54.3001 67.0324) (width 0.25) (layer F.Cu) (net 31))
 (segment (start 54.3001 67.0324) (end 54.3001 72.644) (width 0.25) (layer F.Cu) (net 31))
 (segment (start 52.6227 45.5329) (end 52.6227 44.8383) (width 0.25) (layer B.Cu) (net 8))
 (segment (start 52.6227 44.8383) (end 50.2562 42.4718) (width 0.25) (layer B.Cu) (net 8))
 (segment (start 50.2562 42.4718) (end 50.2562 28.0638) (width 0.25) (layer B.Cu) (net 8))
 (segment (start 50.2562 28.0638) (end 51.224 27.096) (width 0.25) (layer B.Cu) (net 8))
 (segment (start 51.224 27.096) (end 54.5332 27.096) (width 0.25) (layer B.Cu) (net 8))
 (segment (start 54.5332 27.096) (end 59.1792 31.742) (width 0.25) (layer B.Cu) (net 8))
 (segment (start 59.1792 31.742) (end 59.1792 47.7492) (width 0.25) (layer B.Cu) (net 8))
 (segment (start 59.1792 47.7492) (end 60.96 49.53) (width 0.25) (layer B.Cu) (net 8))
 (segment (start 54.1682 45.6032) (end 52.693 45.6032) (width 0.25) (layer B.Cu) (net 8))
 (segment (start 52.693 45.6032) (end 52.6227 45.5329) (width 0.25) (layer B.Cu) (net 8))
 (segment (start 52.6227 45.5329) (end 50.5459 47.6097) (width 0.25) (layer B.Cu) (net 8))
 (segment (start 50.5459 47.6097) (end 50.5459 52.2535) (width 0.25) (layer B.Cu) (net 8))
 (segment (start 54.897 46.609) (end 54.1682 45.8802) (width 0.25) (layer F.Cu) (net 8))
 (segment (start 54.1682 45.8802) (end 54.1682 45.6032) (width 0.25) (layer F.Cu) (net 8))
 (segment (start 50.5459 52.691) (end 51.068 53.2131) (width 0.25) (layer F.Cu) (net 8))
 (segment (start 51.068 53.2131) (end 51.068 53.34) (width 0.25) (layer F.Cu) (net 8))
 (segment (start 45.72 52.691) (end 50.5459 52.691) (width 0.25) (layer F.Cu) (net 8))
 (segment (start 50.5459 52.2535) (end 50.5459 52.691) (width 0.25) (layer F.Cu) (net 8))
 (via (at 54.1682 45.6032) (size 0.8) (layers F.Cu B.Cu) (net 8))
 (via (at 50.5459 52.2535) (size 0.8) (layers F.Cu B.Cu) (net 8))
 (segment (start 52.818 41.8064) (end 50.7065 39.6949) (width 0.25) (layer B.Cu) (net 12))
 (segment (start 50.7065 39.6949) (end 50.7065 28.2504) (width 0.25) (layer B.Cu) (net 12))
 (segment (start 50.7065 28.2504) (end 51.4106 27.5463) (width 0.25) (layer B.Cu) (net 12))
 (segment (start 51.4106 27.5463) (end 54.3466 27.5463) (width 0.25) (layer B.Cu) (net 12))
 (segment (start 54.3466 27.5463) (end 58.6164 31.8161) (width 0.25) (layer B.Cu) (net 12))
 (segment (start 58.6164 31.8161) (end 58.6164 57.3464) (width 0.25) (layer B.Cu) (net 12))
 (segment (start 58.6164 57.3464) (end 60.96 59.69) (width 0.25) (layer B.Cu) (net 12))
 (segment (start 52.818 42.926) (end 52.818 41.8064) (width 0.25) (layer F.Cu) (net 12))
 (via (at 52.818 41.8064) (size 0.8) (layers F.Cu B.Cu) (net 12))
 (segment (start 53.2849 59.182) (end 53.2849 57.3084) (width 0.25) (layer F.Cu) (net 33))
 (segment (start 53.2849 57.3084) (end 53.9513 56.642) (width 0.25) (layer F.Cu) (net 33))
 (segment (start 45.72 41.261) (end 45.8591 41.261) (width 0.25) (layer F.Cu) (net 33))
 (segment (start 45.8591 41.261) (end 52.6979 48.0998) (width 0.25) (layer F.Cu) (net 33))
 (segment (start 52.6979 48.0998) (end 52.6979 51.694) (width 0.25) (layer F.Cu) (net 33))
 (segment (start 52.6979 51.694) (end 53.9513 52.9474) (width 0.25) (layer F.Cu) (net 33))
 (segment (start 53.9513 52.9474) (end 53.9513 56.642) (width 0.25) (layer F.Cu) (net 33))
 (segment (start 53.2849 59.182) (end 54.897 59.182) (width 0.25) (layer F.Cu) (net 33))
 (segment (start 48.989 59.182) (end 53.2849 59.182) (width 0.25) (layer F.Cu) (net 33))
 (segment (start 54.897 56.642) (end 53.9513 56.642) (width 0.25) (layer F.Cu) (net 33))
 (segment (start 48.989 59.182) (end 48.989 60.452) (width 0.25) (layer F.Cu) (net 33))
 (segment (start 54.897 59.182) (end 56.515 59.182) (width 0.25) (layer F.Cu) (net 33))
 (segment (start 56.515 59.182) (end 56.896 59.563) (width 0.25) (layer F.Cu) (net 33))
 (segment (start 56.896 59.563) (end 56.896 60.833) (width 0.25) (layer F.Cu) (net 33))
 (segment (start 56.896 60.833) (end 56.134 61.595) (width 0.25) (layer F.Cu) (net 33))
 (segment (start 56.134 61.595) (end 51.816 61.595) (width 0.25) (layer F.Cu) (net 33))
 (segment (start 51.816 61.595) (end 51.562 61.849) (width 0.25) (layer F.Cu) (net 33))
 (segment (start 51.562 61.849) (end 51.562 63.5) (width 0.25) (layer F.Cu) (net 33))
 (segment (start 51.562 63.5) (end 51.975 63.913) (width 0.25) (layer F.Cu) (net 33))
 (segment (start 51.975 63.913) (end 51.975 65.627) (width 0.25) (layer F.Cu) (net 33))
 (segment (start 51.975 65.627) (end 51.562 66.04) (width 0.25) (layer F.Cu) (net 33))
 (segment (start 51.562 66.04) (end 51.562 71.247) (width 0.25) (layer F.Cu) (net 33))
 (segment (start 51.562 71.247) (end 52.324 72.009) (width 0.25) (layer F.Cu) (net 33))
 (segment (start 52.324 72.009) (end 52.324 73.406) (width 0.25) (layer F.Cu) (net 33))
 (segment (start 52.324 73.406) (end 51.562 74.168) (width 0.25) (layer F.Cu) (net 33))
 (segment (start 51.562 74.168) (end 50.038 74.168) (width 0.25) (layer F.Cu) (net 33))
 (segment (start 50.038 74.168) (end 49.149 73.279) (width 0.25) (layer F.Cu) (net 33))
 (segment (start 49.149 73.279) (end 49.149 71.882) (width 0.25) (layer F.Cu) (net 33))
 (segment (start 49.149 71.882) (end 49.911 71.12) (width 0.25) (layer F.Cu) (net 33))
 (segment (start 49.911 71.12) (end 49.911 66.04) (width 0.25) (layer F.Cu) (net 33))
 (segment (start 49.911 66.04) (end 49.53 65.659) (width 0.25) (layer F.Cu) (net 33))
 (segment (start 49.53 65.659) (end 49.53 64.262) (width 0.25) (layer F.Cu) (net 33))
 (segment (start 49.53 64.262) (end 50.038 63.754) (width 0.25) (layer F.Cu) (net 33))
 (segment (start 50.038 63.754) (end 50.038 62.051) (width 0.25) (layer F.Cu) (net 33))
 (segment (start 50.038 62.051) (end 48.989 61.002) (width 0.25) (layer F.Cu) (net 33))
 (segment (start 48.989 61.002) (end 48.989 60.452) (width 0.25) (layer F.Cu) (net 33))
 (segment (start 54.897 30.861) (end 53.5427 30.861) (width 0.25) (layer F.Cu) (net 11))
 (segment (start 53.5427 30.861) (end 53.5427 27.8457) (width 0.25) (layer F.Cu) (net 11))
 (segment (start 53.5427 27.8457) (end 53.6927 27.6957) (width 0.25) (layer F.Cu) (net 11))
 (segment (start 53.6927 27.6957) (end 56.8055 27.6957) (width 0.25) (layer F.Cu) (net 11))
 (segment (start 56.8055 27.6957) (end 59.6344 30.5246) (width 0.25) (layer F.Cu) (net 11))
 (segment (start 59.6344 30.5246) (end 59.6344 55.8244) (width 0.25) (layer F.Cu) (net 11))
 (segment (start 59.6344 55.8244) (end 60.96 57.15) (width 0.25) (layer F.Cu) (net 11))
 (segment (start 53.7679 40.386) (end 53.7679 44.9778) (width 0.25) (layer F.Cu) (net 37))
 (segment (start 53.7679 44.9778) (end 53.4429 45.3028) (width 0.25) (layer F.Cu) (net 37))
 (segment (start 53.4429 45.3028) (end 53.4429 50.3192) (width 0.25) (layer F.Cu) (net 37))
 (segment (start 53.4429 50.3192) (end 53.5427 50.419) (width 0.25) (layer F.Cu) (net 37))
 (segment (start 54.897 50.419) (end 53.5427 50.419) (width 0.25) (layer F.Cu) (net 37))
 (segment (start 53.7679 40.386) (end 53.5427 40.386) (width 0.25) (layer F.Cu) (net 37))
 (segment (start 54.897 40.386) (end 53.7679 40.386) (width 0.25) (layer F.Cu) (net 37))
 (segment (start 53.0337 30.861) (end 53.0337 31.1671) (width 0.25) (layer F.Cu) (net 37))
 (segment (start 53.0337 31.1671) (end 56.2514 34.3848) (width 0.25) (layer F.Cu) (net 37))
 (segment (start 56.2514 34.3848) (end 56.2514 37.0462) (width 0.25) (layer F.Cu) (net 37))
 (segment (start 56.2514 37.0462) (end 56.0962 37.2014) (width 0.25) (layer F.Cu) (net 37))
 (segment (start 56.0962 37.2014) (end 53.7332 37.2014) (width 0.25) (layer F.Cu) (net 37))
 (segment (start 53.7332 37.2014) (end 53.5427 37.3919) (width 0.25) (layer F.Cu) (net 37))
 (segment (start 53.5427 37.3919) (end 53.5427 40.386) (width 0.25) (layer F.Cu) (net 37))
 (segment (start 53.5427 27.051) (end 53.0337 27.56) (width 0.25) (layer F.Cu) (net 37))
 (segment (start 53.0337 27.56) (end 53.0337 30.861) (width 0.25) (layer F.Cu) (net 37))
 (segment (start 50.3433 30.861) (end 53.0337 30.861) (width 0.25) (layer F.Cu) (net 37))
 (segment (start 54.897 27.051) (end 53.5427 27.051) (width 0.25) (layer F.Cu) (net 37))
 (segment (start 48.989 30.861) (end 50.3433 30.861) (width 0.25) (layer F.Cu) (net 37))
 (segment (start 50.8 64.897) (end 50.8 72.644) (width 0.25) (layer F.Cu) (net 29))
 (segment (start 54.897 60.452) (end 51.943 60.452) (width 0.25) (layer F.Cu) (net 29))
 (segment (start 51.943 60.452) (end 50.8 61.595) (width 0.25) (layer F.Cu) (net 29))
 (segment (start 50.8 61.595) (end 50.8 64.897) (width 0.25) (layer F.Cu) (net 29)))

